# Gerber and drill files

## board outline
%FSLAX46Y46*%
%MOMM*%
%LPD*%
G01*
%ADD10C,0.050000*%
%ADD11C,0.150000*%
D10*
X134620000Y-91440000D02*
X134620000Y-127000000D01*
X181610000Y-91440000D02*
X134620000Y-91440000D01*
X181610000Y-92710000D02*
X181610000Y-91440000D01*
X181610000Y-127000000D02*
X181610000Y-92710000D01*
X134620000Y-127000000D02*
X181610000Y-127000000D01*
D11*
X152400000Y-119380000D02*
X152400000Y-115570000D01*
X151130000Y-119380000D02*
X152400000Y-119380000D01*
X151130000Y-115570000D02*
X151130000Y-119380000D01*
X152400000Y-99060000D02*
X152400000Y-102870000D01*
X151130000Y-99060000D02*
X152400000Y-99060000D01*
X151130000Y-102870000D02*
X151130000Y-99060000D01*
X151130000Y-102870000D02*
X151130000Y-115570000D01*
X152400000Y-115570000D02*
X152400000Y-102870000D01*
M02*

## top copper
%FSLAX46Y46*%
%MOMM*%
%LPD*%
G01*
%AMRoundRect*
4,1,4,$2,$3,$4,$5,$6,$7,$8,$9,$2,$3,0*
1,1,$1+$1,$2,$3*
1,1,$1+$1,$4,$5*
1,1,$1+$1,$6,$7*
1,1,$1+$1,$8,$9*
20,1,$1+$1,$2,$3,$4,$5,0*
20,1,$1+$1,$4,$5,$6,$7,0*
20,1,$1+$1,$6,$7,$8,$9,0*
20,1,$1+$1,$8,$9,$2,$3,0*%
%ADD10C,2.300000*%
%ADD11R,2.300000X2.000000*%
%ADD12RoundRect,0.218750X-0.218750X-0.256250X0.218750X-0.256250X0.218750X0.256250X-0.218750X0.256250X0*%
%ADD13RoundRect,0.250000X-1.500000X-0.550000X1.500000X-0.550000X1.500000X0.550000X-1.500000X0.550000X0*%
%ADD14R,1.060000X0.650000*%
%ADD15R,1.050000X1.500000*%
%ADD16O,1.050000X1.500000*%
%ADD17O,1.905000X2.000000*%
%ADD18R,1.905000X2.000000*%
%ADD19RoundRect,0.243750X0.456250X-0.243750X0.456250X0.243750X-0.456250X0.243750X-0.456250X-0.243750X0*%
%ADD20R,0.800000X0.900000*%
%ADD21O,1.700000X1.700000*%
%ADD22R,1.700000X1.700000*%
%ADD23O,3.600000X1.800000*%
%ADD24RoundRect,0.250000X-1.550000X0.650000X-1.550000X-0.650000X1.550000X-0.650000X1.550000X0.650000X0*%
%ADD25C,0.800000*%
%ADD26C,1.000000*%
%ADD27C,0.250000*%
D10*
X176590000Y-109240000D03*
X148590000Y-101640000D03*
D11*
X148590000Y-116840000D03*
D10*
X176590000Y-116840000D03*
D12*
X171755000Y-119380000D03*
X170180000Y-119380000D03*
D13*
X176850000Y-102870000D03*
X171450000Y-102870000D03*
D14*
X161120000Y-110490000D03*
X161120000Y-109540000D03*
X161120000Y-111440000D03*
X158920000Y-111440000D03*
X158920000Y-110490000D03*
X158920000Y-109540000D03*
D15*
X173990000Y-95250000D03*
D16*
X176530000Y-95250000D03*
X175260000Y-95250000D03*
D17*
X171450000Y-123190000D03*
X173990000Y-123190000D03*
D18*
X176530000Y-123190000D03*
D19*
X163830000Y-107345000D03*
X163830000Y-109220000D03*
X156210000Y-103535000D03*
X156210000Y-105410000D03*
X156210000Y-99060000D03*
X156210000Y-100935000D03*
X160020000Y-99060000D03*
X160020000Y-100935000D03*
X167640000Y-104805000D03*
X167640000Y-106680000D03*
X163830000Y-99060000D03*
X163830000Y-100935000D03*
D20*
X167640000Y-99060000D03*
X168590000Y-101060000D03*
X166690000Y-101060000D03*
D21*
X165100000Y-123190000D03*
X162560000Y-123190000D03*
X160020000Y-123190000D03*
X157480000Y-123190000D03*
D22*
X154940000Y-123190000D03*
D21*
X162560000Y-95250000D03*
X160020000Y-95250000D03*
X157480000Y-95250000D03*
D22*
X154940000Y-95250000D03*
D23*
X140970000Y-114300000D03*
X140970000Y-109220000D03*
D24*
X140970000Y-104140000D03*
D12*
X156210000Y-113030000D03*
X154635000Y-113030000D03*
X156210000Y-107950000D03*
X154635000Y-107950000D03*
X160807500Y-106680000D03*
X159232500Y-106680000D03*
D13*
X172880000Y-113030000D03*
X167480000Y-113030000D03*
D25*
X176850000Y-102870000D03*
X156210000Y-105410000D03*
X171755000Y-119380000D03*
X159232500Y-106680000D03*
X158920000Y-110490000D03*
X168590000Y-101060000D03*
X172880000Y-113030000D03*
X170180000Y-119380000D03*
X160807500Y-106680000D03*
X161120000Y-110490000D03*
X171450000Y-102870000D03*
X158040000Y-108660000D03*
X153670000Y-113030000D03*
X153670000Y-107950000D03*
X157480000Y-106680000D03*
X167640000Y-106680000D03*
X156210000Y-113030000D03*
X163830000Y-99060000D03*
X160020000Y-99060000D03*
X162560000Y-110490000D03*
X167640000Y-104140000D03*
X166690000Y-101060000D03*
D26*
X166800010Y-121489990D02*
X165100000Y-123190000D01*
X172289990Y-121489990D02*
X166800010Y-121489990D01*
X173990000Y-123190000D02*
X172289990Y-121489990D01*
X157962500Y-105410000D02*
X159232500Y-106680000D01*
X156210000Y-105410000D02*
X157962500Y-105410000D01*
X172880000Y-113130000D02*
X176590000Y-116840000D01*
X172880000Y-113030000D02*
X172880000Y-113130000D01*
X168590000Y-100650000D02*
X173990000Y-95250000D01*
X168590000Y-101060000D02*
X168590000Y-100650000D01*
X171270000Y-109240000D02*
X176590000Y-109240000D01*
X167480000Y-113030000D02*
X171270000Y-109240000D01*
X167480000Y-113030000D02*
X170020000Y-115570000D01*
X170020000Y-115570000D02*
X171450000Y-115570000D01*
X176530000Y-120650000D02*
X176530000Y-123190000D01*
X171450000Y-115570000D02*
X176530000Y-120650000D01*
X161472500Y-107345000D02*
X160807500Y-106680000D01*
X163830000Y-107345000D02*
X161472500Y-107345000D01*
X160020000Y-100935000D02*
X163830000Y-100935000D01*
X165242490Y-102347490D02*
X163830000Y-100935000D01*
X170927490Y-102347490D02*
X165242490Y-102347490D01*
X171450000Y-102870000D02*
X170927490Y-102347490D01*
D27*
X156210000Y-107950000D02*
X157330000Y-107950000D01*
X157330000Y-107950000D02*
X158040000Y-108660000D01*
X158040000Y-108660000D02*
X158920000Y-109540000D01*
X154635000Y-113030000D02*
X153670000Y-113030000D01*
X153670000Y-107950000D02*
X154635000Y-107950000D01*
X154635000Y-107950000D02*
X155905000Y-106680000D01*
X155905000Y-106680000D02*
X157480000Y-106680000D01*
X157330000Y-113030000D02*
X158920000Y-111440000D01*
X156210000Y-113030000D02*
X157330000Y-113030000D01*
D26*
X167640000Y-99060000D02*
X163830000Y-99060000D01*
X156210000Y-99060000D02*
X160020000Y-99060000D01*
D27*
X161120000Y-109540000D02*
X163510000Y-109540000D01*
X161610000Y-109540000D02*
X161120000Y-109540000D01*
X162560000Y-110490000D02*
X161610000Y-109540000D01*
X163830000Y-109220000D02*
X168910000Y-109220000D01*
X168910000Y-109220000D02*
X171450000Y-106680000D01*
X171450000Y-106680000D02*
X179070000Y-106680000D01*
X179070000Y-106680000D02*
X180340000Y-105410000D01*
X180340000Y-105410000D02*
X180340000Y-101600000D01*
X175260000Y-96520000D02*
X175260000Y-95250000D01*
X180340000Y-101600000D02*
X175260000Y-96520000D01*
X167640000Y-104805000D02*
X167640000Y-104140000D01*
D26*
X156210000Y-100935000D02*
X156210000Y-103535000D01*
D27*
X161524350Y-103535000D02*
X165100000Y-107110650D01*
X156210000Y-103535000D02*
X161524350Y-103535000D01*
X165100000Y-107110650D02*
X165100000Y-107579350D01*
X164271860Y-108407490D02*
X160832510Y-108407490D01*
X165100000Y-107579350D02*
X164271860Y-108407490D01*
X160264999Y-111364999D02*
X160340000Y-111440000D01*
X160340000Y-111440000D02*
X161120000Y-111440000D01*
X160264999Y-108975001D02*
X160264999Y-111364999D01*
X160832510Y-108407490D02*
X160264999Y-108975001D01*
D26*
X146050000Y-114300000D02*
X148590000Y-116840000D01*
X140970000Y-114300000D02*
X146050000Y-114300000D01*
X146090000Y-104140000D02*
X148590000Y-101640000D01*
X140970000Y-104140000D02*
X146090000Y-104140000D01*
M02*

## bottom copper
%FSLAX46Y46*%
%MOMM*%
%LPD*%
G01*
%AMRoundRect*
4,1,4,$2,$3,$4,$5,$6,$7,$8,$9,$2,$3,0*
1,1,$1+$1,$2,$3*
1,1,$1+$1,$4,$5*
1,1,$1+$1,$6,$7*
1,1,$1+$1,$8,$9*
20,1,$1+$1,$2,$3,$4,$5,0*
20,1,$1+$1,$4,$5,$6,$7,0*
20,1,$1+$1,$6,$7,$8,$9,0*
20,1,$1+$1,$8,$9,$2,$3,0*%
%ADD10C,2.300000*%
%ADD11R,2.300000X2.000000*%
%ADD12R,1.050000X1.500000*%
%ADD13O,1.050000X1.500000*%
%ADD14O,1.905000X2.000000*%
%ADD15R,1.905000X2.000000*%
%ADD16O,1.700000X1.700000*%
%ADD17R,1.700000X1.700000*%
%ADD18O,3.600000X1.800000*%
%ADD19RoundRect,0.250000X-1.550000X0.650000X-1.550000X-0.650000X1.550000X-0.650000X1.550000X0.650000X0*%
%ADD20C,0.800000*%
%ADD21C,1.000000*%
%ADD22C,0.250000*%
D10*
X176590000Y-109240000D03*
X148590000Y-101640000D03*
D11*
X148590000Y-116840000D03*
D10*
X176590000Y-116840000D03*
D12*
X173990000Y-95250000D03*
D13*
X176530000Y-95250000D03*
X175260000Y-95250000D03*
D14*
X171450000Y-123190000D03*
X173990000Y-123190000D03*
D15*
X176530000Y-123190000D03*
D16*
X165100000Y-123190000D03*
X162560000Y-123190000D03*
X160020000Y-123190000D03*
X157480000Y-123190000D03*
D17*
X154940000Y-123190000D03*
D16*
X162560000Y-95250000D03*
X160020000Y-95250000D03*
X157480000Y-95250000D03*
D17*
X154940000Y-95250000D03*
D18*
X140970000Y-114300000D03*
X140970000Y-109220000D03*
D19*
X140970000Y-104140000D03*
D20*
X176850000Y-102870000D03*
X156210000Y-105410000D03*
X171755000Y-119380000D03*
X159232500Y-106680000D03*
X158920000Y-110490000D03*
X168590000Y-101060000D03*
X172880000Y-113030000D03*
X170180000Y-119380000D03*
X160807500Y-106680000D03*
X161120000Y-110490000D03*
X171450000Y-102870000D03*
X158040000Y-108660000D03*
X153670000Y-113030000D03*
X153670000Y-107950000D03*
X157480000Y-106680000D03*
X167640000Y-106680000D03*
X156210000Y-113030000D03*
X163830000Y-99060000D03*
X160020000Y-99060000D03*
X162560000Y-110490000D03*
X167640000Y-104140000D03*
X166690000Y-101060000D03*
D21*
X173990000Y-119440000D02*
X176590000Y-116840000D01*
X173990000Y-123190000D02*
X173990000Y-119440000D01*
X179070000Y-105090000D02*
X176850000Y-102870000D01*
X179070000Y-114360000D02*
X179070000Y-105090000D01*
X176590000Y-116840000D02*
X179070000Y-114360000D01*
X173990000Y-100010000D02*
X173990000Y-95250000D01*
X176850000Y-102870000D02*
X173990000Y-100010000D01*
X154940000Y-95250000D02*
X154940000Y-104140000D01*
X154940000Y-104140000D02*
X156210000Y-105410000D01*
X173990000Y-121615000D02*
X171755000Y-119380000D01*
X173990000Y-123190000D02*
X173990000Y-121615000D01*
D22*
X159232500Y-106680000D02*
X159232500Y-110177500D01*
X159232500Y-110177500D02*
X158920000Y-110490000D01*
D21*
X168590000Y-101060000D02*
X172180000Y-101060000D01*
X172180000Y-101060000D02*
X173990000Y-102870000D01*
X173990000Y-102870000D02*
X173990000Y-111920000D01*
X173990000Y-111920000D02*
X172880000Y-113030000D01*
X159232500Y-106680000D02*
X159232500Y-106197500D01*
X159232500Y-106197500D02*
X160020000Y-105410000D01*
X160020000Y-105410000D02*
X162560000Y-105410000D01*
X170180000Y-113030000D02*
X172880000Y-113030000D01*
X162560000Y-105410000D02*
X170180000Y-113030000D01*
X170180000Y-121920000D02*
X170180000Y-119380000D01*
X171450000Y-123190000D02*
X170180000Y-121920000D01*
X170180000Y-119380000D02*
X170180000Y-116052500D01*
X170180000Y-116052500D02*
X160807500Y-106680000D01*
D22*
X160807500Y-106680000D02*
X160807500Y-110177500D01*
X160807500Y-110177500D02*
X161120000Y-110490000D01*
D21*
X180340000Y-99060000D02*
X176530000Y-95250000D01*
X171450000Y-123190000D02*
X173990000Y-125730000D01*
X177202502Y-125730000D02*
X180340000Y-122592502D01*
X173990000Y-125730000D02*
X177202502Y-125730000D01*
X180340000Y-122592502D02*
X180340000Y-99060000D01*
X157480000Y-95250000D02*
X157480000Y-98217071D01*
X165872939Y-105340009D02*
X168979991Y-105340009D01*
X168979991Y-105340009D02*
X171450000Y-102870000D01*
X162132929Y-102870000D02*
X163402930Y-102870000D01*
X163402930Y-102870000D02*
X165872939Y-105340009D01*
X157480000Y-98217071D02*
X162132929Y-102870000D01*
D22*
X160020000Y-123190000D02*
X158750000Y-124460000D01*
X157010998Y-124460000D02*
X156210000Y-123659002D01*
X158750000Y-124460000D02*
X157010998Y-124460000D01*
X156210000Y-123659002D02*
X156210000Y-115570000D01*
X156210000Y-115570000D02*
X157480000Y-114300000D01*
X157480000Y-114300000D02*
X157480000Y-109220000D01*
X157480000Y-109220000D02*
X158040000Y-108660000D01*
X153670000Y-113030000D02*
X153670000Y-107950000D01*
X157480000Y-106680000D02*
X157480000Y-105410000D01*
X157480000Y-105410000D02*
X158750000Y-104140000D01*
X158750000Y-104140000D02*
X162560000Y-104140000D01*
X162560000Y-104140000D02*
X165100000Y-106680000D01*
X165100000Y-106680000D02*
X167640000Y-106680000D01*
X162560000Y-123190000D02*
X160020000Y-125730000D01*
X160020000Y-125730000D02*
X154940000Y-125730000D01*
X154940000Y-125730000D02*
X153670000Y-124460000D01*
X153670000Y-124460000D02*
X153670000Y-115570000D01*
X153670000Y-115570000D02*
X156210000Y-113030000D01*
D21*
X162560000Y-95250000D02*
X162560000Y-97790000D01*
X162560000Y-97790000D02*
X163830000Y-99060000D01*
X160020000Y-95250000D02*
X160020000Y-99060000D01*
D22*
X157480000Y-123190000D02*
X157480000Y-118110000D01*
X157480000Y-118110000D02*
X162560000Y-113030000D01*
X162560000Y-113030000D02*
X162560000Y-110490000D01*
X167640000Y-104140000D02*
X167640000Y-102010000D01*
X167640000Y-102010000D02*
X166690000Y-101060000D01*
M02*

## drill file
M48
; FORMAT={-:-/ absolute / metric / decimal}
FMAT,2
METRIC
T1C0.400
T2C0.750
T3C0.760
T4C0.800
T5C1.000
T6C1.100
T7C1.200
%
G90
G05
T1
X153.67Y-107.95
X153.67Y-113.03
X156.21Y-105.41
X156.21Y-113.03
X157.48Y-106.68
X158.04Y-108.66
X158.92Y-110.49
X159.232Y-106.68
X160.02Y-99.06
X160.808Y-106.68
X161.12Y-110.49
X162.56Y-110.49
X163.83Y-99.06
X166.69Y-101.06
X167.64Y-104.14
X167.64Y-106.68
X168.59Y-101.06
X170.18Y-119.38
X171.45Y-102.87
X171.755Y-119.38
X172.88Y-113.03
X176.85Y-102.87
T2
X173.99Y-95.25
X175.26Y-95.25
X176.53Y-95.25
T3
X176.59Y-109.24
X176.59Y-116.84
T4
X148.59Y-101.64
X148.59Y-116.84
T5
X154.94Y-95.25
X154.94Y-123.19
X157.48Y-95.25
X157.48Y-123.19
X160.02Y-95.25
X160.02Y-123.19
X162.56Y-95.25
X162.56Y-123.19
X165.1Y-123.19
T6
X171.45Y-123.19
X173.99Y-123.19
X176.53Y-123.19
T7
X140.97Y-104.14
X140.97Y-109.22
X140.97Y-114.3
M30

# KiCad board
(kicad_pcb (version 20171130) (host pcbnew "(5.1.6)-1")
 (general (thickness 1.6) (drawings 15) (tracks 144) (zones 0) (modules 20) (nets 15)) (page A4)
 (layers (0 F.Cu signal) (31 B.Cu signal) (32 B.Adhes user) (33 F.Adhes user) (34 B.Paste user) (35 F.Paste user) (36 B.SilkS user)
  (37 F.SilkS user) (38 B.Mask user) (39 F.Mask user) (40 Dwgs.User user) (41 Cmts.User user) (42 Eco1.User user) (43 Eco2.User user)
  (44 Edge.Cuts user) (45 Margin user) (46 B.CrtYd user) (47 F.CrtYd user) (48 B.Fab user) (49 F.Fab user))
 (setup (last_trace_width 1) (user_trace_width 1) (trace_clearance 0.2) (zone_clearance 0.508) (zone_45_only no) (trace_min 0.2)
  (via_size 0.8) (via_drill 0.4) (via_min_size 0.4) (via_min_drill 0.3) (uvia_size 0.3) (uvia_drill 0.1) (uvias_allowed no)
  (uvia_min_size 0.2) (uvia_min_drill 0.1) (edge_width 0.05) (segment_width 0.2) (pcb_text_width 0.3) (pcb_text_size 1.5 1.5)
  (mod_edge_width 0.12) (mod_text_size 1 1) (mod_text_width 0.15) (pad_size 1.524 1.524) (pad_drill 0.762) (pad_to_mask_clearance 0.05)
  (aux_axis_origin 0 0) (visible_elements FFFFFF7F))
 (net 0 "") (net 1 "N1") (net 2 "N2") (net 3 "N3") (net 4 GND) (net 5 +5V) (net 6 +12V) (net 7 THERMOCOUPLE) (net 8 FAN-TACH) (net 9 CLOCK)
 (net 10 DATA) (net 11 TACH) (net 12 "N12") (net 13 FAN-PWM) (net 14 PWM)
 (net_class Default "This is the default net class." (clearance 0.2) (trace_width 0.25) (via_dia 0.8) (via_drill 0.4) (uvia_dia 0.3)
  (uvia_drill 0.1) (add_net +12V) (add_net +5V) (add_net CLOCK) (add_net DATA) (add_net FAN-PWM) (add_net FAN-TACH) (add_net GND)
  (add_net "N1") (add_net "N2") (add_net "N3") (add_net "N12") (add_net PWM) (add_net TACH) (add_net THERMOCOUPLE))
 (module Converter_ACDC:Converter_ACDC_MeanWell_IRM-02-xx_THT (layer B.Cu) (at 148.59 116.84)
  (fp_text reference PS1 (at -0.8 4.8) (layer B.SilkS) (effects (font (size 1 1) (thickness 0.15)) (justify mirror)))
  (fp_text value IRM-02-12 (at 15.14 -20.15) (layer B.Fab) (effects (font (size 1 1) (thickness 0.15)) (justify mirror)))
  (pad 4 thru_hole circle (at 28 -7.6) (size 2.3 2.3) (drill 0.76) (layers *.Cu *.Mask) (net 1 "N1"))
  (pad 2 thru_hole circle (at 0 -15.2) (size 2.3 2.3) (drill 0.8) (layers *.Cu *.Mask) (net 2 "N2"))
  (pad 1 thru_hole rect (at 0 0) (size 2.3 2) (drill 0.8) (layers *.Cu *.Mask) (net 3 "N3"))
  (pad 3 thru_hole circle (at 28 0) (size 2.3 2.3) (drill 0.76) (layers *.Cu *.Mask) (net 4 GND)))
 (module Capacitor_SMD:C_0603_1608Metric (layer F.Cu) (at 170.9675 119.38)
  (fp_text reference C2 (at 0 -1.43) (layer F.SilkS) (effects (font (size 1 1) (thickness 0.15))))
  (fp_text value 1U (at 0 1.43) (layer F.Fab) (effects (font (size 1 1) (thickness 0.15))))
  (pad 2 smd roundrect (at 0.7875 0) (size 0.875 0.95) (layers F.Cu F.Paste F.Mask) (roundrect_rratio 0.25) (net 4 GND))
  (pad 1 smd roundrect (at -0.7875 0) (size 0.875 0.95) (layers F.Cu F.Paste F.Mask) (roundrect_rratio 0.25) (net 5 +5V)))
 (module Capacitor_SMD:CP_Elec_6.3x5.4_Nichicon (layer F.Cu) (at 174.15 102.87)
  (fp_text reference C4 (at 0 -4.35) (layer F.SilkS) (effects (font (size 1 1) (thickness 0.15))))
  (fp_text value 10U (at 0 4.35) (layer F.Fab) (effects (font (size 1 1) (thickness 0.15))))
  (pad 2 smd roundrect (at 2.7 0) (size 3.5 1.6) (layers F.Cu F.Paste F.Mask) (roundrect_rratio 0.15625) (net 4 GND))
  (pad 1 smd roundrect (at -2.7 0) (size 3.5 1.6) (layers F.Cu F.Paste F.Mask) (roundrect_rratio 0.15625) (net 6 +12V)))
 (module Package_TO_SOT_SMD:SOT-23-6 (layer F.Cu) (at 160.02 110.49)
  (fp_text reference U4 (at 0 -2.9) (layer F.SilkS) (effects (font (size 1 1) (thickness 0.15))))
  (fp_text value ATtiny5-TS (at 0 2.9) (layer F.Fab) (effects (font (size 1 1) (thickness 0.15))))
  (pad 5 smd rect (at 1.1 0) (size 1.06 0.65) (layers F.Cu F.Paste F.Mask) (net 5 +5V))
  (pad 6 smd rect (at 1.1 -0.95) (size 1.06 0.65) (layers F.Cu F.Paste F.Mask) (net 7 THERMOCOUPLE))
  (pad 4 smd rect (at 1.1 0.95) (size 1.06 0.65) (layers F.Cu F.Paste F.Mask) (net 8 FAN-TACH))
  (pad 3 smd rect (at -1.1 0.95) (size 1.06 0.65) (layers F.Cu F.Paste F.Mask) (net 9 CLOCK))
  (pad 2 smd rect (at -1.1 0) (size 1.06 0.65) (layers F.Cu F.Paste F.Mask) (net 4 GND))
  (pad 1 smd rect (at -1.1 -0.95) (size 1.06 0.65) (layers F.Cu F.Paste F.Mask) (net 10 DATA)))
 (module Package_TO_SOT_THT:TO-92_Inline (layer F.Cu) (at 173.99 95.25)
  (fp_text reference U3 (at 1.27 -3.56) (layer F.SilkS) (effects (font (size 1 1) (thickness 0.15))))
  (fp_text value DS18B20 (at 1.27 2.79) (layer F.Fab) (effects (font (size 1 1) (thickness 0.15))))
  (pad 1 thru_hole rect (at 0 0) (size 1.05 1.5) (drill 0.75) (layers *.Cu *.Mask) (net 4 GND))
  (pad 3 thru_hole oval (at 2.54 0) (size 1.05 1.5) (drill 0.75) (layers *.Cu *.Mask) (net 5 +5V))
  (pad 2 thru_hole oval (at 1.27 0) (size 1.05 1.5) (drill 0.75) (layers *.Cu *.Mask) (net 7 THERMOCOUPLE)))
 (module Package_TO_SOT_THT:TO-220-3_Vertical (layer F.Cu) (at 176.53 123.19 180)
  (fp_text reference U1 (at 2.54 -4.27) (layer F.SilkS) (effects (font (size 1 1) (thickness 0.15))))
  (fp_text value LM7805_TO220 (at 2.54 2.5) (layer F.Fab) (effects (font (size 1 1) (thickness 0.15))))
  (pad 3 thru_hole oval (at 5.08 0 180) (size 1.905 2) (drill 1.1) (layers *.Cu *.Mask) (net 5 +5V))
  (pad 2 thru_hole oval (at 2.54 0 180) (size 1.905 2) (drill 1.1) (layers *.Cu *.Mask) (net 4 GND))
  (pad 1 thru_hole rect (at 0 0 180) (size 1.905 2) (drill 1.1) (layers *.Cu *.Mask) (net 1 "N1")))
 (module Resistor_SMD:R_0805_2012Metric (layer F.Cu) (at 163.83 108.2825 90)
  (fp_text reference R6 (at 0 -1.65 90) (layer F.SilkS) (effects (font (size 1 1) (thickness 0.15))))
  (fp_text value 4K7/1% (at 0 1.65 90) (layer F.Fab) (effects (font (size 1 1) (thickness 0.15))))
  (pad 2 smd roundrect (at 0.9375 0 90) (size 0.975 1.4) (layers F.Cu F.Paste F.Mask) (roundrect_rratio 0.25) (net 5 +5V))
  (pad 1 smd roundrect (at -0.9375 0 90) (size 0.975 1.4) (layers F.Cu F.Paste F.Mask) (roundrect_rratio 0.25) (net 7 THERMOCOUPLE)))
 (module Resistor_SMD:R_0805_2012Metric (layer F.Cu) (at 156.21 104.4725 90)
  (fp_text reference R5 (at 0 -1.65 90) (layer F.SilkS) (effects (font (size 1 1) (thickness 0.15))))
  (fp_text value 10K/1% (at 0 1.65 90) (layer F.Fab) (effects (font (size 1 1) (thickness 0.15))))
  (pad 2 smd roundrect (at 0.9375 0 90) (size 0.975 1.4) (layers F.Cu F.Paste F.Mask) (roundrect_rratio 0.25) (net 8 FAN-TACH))
  (pad 1 smd roundrect (at -0.9375 0 90) (size 0.975 1.4) (layers F.Cu F.Paste F.Mask) (roundrect_rratio 0.25) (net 4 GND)))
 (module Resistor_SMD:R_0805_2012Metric (layer F.Cu) (at 156.21 99.9975 90)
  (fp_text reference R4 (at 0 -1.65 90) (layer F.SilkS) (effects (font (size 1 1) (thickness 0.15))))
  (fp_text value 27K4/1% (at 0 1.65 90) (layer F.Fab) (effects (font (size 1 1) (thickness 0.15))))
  (pad 2 smd roundrect (at 0.9375 0 90) (size 0.975 1.4) (layers F.Cu F.Paste F.Mask) (roundrect_rratio 0.25) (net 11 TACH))
  (pad 1 smd roundrect (at -0.9375 0 90) (size 0.975 1.4) (layers F.Cu F.Paste F.Mask) (roundrect_rratio 0.25) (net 8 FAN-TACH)))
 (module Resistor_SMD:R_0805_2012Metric (layer F.Cu) (at 160.02 99.9975 90)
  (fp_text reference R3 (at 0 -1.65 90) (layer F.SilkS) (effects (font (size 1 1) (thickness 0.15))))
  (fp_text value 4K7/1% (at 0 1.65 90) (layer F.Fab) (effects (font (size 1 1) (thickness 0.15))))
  (pad 2 smd roundrect (at 0.9375 0 90) (size 0.975 1.4) (layers F.Cu F.Paste F.Mask) (roundrect_rratio 0.25) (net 11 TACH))
  (pad 1 smd roundrect (at -0.9375 0 90) (size 0.975 1.4) (layers F.Cu F.Paste F.Mask) (roundrect_rratio 0.25) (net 6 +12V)))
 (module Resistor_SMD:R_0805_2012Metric (layer F.Cu) (at 167.64 105.7425 90)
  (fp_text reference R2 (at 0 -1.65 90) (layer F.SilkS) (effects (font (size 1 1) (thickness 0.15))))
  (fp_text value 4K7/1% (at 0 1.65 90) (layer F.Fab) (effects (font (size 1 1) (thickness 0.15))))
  (pad 2 smd roundrect (at 0.9375 0 90) (size 0.975 1.4) (layers F.Cu F.Paste F.Mask) (roundrect_rratio 0.25) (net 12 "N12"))
  (pad 1 smd roundrect (at -0.9375 0 90) (size 0.975 1.4) (layers F.Cu F.Paste F.Mask) (roundrect_rratio 0.25) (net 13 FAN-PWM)))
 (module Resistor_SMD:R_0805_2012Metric (layer F.Cu) (at 163.83 99.9975 90)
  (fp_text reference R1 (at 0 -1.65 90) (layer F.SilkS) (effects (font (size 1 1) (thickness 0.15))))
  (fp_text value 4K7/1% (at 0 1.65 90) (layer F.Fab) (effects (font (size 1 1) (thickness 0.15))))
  (pad 2 smd roundrect (at 0.9375 0 90) (size 0.975 1.4) (layers F.Cu F.Paste F.Mask) (roundrect_rratio 0.25) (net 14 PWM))
  (pad 1 smd roundrect (at -0.9375 0 90) (size 0.975 1.4) (layers F.Cu F.Paste F.Mask) (roundrect_rratio 0.25) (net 6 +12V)))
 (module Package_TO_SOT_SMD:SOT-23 (layer F.Cu) (at 167.64 100.06 90)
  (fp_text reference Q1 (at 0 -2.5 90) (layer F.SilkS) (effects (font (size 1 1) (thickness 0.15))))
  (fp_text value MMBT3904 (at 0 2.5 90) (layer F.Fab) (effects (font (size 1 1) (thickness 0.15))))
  (pad 3 smd rect (at 1 0 90) (size 0.9 0.8) (layers F.Cu F.Paste F.Mask) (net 14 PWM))
  (pad 2 smd rect (at -1 0.95 90) (size 0.9 0.8) (layers F.Cu F.Paste F.Mask) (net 4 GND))
  (pad 1 smd rect (at -1 -0.95 90) (size 0.9 0.8) (layers F.Cu F.Paste F.Mask) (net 12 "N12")))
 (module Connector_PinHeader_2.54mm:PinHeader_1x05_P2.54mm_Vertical (layer F.Cu) (at 154.94 123.19 90)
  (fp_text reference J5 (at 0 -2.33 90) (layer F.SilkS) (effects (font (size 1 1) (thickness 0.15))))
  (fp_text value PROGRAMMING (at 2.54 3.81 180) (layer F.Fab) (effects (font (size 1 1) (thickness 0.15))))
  (pad 5 thru_hole oval (at 0 10.16 90) (size 1.7 1.7) (drill 1) (layers *.Cu *.Mask) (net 4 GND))
  (pad 4 thru_hole oval (at 0 7.62 90) (size 1.7 1.7) (drill 1) (layers *.Cu *.Mask) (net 9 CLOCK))
  (pad 3 thru_hole oval (at 0 5.08 90) (size 1.7 1.7) (drill 1) (layers *.Cu *.Mask) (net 10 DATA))
  (pad 2 thru_hole oval (at 0 2.54 90) (size 1.7 1.7) (drill 1) (layers *.Cu *.Mask) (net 7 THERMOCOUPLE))
  (pad 1 thru_hole rect (at 0 0 90) (size 1.7 1.7) (drill 1) (layers *.Cu *.Mask)))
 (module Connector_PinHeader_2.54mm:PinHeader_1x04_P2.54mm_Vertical (layer F.Cu) (at 154.94 95.25 90)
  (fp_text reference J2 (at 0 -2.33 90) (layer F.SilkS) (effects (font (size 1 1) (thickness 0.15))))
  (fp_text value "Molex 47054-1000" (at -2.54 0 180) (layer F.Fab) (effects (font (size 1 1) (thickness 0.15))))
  (pad 4 thru_hole oval (at 0 7.62 90) (size 1.7 1.7) (drill 1) (layers *.Cu *.Mask) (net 14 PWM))
  (pad 3 thru_hole oval (at 0 5.08 90) (size 1.7 1.7) (drill 1) (layers *.Cu *.Mask) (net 11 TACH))
  (pad 2 thru_hole oval (at 0 2.54 90) (size 1.7 1.7) (drill 1) (layers *.Cu *.Mask) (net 6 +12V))
  (pad 1 thru_hole rect (at 0 0 90) (size 1.7 1.7) (drill 1) (layers *.Cu *.Mask) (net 4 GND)))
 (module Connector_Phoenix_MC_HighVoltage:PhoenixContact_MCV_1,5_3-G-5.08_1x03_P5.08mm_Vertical (layer B.Cu) (at 140.97 104.14 270)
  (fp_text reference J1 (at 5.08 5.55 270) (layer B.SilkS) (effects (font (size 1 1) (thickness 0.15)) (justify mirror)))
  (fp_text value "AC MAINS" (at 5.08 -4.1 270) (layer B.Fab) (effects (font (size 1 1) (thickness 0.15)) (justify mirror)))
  (pad 3 thru_hole oval (at 10.16 0 270) (size 1.8 3.6) (drill 1.2) (layers *.Cu *.Mask) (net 3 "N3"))
  (pad 2 thru_hole oval (at 5.08 0 270) (size 1.8 3.6) (drill 1.2) (layers *.Cu *.Mask))
  (pad 1 thru_hole roundrect (at 0 0 270) (size 1.8 3.6) (drill 1.2) (layers *.Cu *.Mask) (roundrect_rratio 0.138889) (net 2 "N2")))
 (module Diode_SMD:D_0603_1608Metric (layer F.Cu) (at 155.4225 113.03)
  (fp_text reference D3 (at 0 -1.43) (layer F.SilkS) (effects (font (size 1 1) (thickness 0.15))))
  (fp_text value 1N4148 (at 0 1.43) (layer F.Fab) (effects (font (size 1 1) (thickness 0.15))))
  (pad 2 smd roundrect (at 0.7875 0) (size 0.875 0.95) (layers F.Cu F.Paste F.Mask) (roundrect_rratio 0.25) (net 9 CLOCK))
  (pad 1 smd roundrect (at -0.7875 0) (size 0.875 0.95) (layers F.Cu F.Paste F.Mask) (roundrect_rratio 0.25) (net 13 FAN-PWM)))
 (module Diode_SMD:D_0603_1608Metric (layer F.Cu) (at 155.4225 107.95)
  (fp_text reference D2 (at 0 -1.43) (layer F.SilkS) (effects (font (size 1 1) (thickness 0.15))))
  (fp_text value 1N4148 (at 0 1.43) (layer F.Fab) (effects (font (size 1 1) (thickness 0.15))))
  (pad 2 smd roundrect (at 0.7875 0) (size 0.875 0.95) (layers F.Cu F.Paste F.Mask) (roundrect_rratio 0.25) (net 10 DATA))
  (pad 1 smd roundrect (at -0.7875 0) (size 0.875 0.95) (layers F.Cu F.Paste F.Mask) (roundrect_rratio 0.25) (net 13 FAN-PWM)))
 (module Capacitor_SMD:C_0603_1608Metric (layer F.Cu) (at 160.02 106.68)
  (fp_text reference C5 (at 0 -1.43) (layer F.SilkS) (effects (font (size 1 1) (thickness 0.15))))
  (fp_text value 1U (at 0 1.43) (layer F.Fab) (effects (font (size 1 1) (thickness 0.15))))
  (pad 2 smd roundrect (at 0.7875 0) (size 0.875 0.95) (layers F.Cu F.Paste F.Mask) (roundrect_rratio 0.25) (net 5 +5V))
  (pad 1 smd roundrect (at -0.7875 0) (size 0.875 0.95) (layers F.Cu F.Paste F.Mask) (roundrect_rratio 0.25) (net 4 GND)))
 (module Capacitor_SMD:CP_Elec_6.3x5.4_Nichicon (layer F.Cu) (at 170.18 113.03)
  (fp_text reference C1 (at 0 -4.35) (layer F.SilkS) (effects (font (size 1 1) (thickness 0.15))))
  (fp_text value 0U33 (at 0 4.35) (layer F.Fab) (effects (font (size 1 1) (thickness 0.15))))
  (pad 2 smd roundrect (at 2.7 0) (size 3.5 1.6) (layers F.Cu F.Paste F.Mask) (roundrect_rratio 0.15625) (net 4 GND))
  (pad 1 smd roundrect (at -2.7 0) (size 3.5 1.6) (layers F.Cu F.Paste F.Mask) (roundrect_rratio 0.15625) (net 1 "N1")))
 (gr_line (start 134.62 91.44) (end 134.62 127) (layer Edge.Cuts) (width 0.05))
 (gr_line (start 181.61 91.44) (end 134.62 91.44) (layer Edge.Cuts) (width 0.05))
 (gr_line (start 181.61 92.71) (end 181.61 91.44) (layer Edge.Cuts) (width 0.05))
 (gr_line (start 181.61 127) (end 181.61 92.71) (layer Edge.Cuts) (width 0.05))
 (gr_line (start 134.62 127) (end 181.61 127) (layer Edge.Cuts) (width 0.05))
 (gr_line (start 152.4 119.38) (end 152.4 115.57) (layer Edge.Cuts) (width 0.15))
 (gr_line (start 151.13 119.38) (end 152.4 119.38) (layer Edge.Cuts) (width 0.15))
 (gr_line (start 151.13 115.57) (end 151.13 119.38) (layer Edge.Cuts) (width 0.15))
 (gr_line (start 152.4 99.06) (end 152.4 102.87) (layer Edge.Cuts) (width 0.15))
 (gr_line (start 151.13 99.06) (end 152.4 99.06) (layer Edge.Cuts) (width 0.15))
 (gr_line (start 151.13 102.87) (end 151.13 99.06) (layer Edge.Cuts) (width 0.15))
 (gr_line (start 151.13 102.87) (end 151.13 115.57) (layer Edge.Cuts) (width 0.15))
 (gr_line (start 152.4 115.57) (end 152.4 102.87) (layer Edge.Cuts) (width 0.15))
 (segment (start 173.99 119.44) (end 176.59 116.84) (width 1) (layer B.Cu) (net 4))
 (segment (start 173.99 123.19) (end 173.99 119.44) (width 1) (layer B.Cu) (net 4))
 (segment (start 166.80001 121.48999) (end 165.1 123.19) (width 1) (layer F.Cu) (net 4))
 (segment (start 172.28999 121.48999) (end 166.80001 121.48999) (width 1) (layer F.Cu) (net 4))
 (segment (start 173.99 123.19) (end 172.28999 121.48999) (width 1) (layer F.Cu) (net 4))
 (segment (start 179.07 105.09) (end 176.85 102.87) (width 1) (layer B.Cu) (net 4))
 (segment (start 179.07 114.36) (end 179.07 105.09) (width 1) (layer B.Cu) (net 4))
 (segment (start 176.59 116.84) (end 179.07 114.36) (width 1) (layer B.Cu) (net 4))
 (via (at 176.85 102.87) (size 0.8) (drill 0.4) (layers F.Cu B.Cu) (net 4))
 (segment (start 173.99 100.01) (end 173.99 95.25) (width 1) (layer B.Cu) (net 4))
 (segment (start 176.85 102.87) (end 173.99 100.01) (width 1) (layer B.Cu) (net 4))
 (via (at 156.21 105.41) (size 0.8) (drill 0.4) (layers F.Cu B.Cu) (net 4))
 (segment (start 154.94 95.25) (end 154.94 104.14) (width 1) (layer B.Cu) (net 4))
 (segment (start 154.94 104.14) (end 156.21 105.41) (width 1) (layer B.Cu) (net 4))
 (segment (start 157.9625 105.41) (end 159.2325 106.68) (width 1) (layer F.Cu) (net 4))
 (segment (start 156.21 105.41) (end 157.9625 105.41) (width 1) (layer F.Cu) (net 4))
 (segment (start 173.99 121.615) (end 171.755 119.38) (width 1) (layer B.Cu) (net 4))
 (via (at 171.755 119.38) (size 0.8) (drill 0.4) (layers F.Cu B.Cu) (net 4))
 (segment (start 173.99 123.19) (end 173.99 121.615) (width 1) (layer B.Cu) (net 4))
 (segment (start 172.88 113.13) (end 176.59 116.84) (width 1) (layer F.Cu) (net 4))
 (segment (start 172.88 113.03) (end 172.88 113.13) (width 1) (layer F.Cu) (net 4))
 (segment (start 168.59 100.65) (end 173.99 95.25) (width 1) (layer F.Cu) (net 4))
 (segment (start 168.59 101.06) (end 168.59 100.65) (width 1) (layer F.Cu) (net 4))
 (via (at 159.2325 106.68) (size 0.8) (drill 0.4) (layers F.Cu B.Cu) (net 4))
 (segment (start 159.2325 106.68) (end 159.2325 110.1775) (width 0.25) (layer B.Cu) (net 4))
 (via (at 158.92 110.49) (size 0.8) (drill 0.4) (layers F.Cu B.Cu) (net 4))
 (segment (start 159.2325 110.1775) (end 158.92 110.49) (width 0.25) (layer B.Cu) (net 4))
 (via (at 168.59 101.06) (size 0.8) (drill 0.4) (layers F.Cu B.Cu) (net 4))
 (segment (start 168.59 101.06) (end 172.18 101.06) (width 1) (layer B.Cu) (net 4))
 (segment (start 172.18 101.06) (end 173.99 102.87) (width 1) (layer B.Cu) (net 4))
 (via (at 172.88 113.03) (size 0.8) (drill 0.4) (layers F.Cu B.Cu) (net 4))
 (segment (start 173.99 102.87) (end 173.99 111.92) (width 1) (layer B.Cu) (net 4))
 (segment (start 173.99 111.92) (end 172.88 113.03) (width 1) (layer B.Cu) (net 4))
 (segment (start 159.2325 106.68) (end 159.2325 106.1975) (width 1) (layer B.Cu) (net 4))
 (segment (start 159.2325 106.1975) (end 160.02 105.41) (width 1) (layer B.Cu) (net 4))
 (segment (start 160.02 105.41) (end 162.56 105.41) (width 1) (layer B.Cu) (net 4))
 (segment (start 170.18 113.03) (end 172.88 113.03) (width 1) (layer B.Cu) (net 4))
 (segment (start 162.56 105.41) (end 170.18 113.03) (width 1) (layer B.Cu) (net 4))
 (segment (start 171.27 109.24) (end 176.59 109.24) (width 1) (layer F.Cu) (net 1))
 (segment (start 167.48 113.03) (end 171.27 109.24) (width 1) (layer F.Cu) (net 1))
 (segment (start 167.48 113.03) (end 170.02 115.57) (width 1) (layer F.Cu) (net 1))
 (segment (start 170.02 115.57) (end 171.45 115.57) (width 1) (layer F.Cu) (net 1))
 (segment (start 176.53 120.65) (end 176.53 123.19) (width 1) (layer F.Cu) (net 1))
 (segment (start 171.45 115.57) (end 176.53 120.65) (width 1) (layer F.Cu) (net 1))
 (segment (start 161.4725 107.345) (end 160.8075 106.68) (width 1) (layer F.Cu) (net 5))
 (segment (start 163.83 107.345) (end 161.4725 107.345) (width 1) (layer F.Cu) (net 5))
 (via (at 170.18 119.38) (size 0.8) (drill 0.4) (layers F.Cu B.Cu) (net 5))
 (segment (start 170.18 121.92) (end 170.18 119.38) (width 1) (layer B.Cu) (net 5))
 (segment (start 171.45 123.19) (end 170.18 121.92) (width 1) (layer B.Cu) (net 5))
 (via (at 160.8075 106.68) (size 0.8) (drill 0.4) (layers F.Cu B.Cu) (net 5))
 (segment (start 170.18 119.38) (end 170.18 116.0525) (width 1) (layer B.Cu) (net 5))
 (segment (start 170.18 116.0525) (end 160.8075 106.68) (width 1) (layer B.Cu) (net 5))
 (via (at 161.12 110.49) (size 0.8) (drill 0.4) (layers F.Cu B.Cu) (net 5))
 (segment (start 160.8075 106.68) (end 160.8075 110.1775) (width 0.25) (layer B.Cu) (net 5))
 (segment (start 160.8075 110.1775) (end 161.12 110.49) (width 0.25) (layer B.Cu) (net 5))
 (segment (start 180.34 99.06) (end 176.53 95.25) (width 1) (layer B.Cu) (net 5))
 (segment (start 171.45 123.19) (end 173.99 125.73) (width 1) (layer B.Cu) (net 5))
 (segment (start 177.202502 125.73) (end 180.34 122.592502) (width 1) (layer B.Cu) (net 5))
 (segment (start 173.99 125.73) (end 177.202502 125.73) (width 1) (layer B.Cu) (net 5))
 (segment (start 180.34 122.592502) (end 180.34 99.06) (width 1) (layer B.Cu) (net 5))
 (segment (start 160.02 100.935) (end 163.83 100.935) (width 1) (layer F.Cu) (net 6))
 (segment (start 165.24249 102.34749) (end 163.83 100.935) (width 1) (layer F.Cu) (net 6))
 (segment (start 170.92749 102.34749) (end 165.24249 102.34749) (width 1) (layer F.Cu) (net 6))
 (segment (start 171.45 102.87) (end 170.92749 102.34749) (width 1) (layer F.Cu) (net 6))
 (via (at 171.45 102.87) (size 0.8) (drill 0.4) (layers F.Cu B.Cu) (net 6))
 (segment (start 157.48 95.25) (end 157.48 98.217071) (width 1) (layer B.Cu) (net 6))
 (segment (start 165.872939 105.340009) (end 168.979991 105.340009) (width 1) (layer B.Cu) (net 6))
 (segment (start 168.979991 105.340009) (end 171.45 102.87) (width 1) (layer B.Cu) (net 6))
 (segment (start 162.132929 102.87) (end 163.40293 102.87) (width 1) (layer B.Cu) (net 6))
 (segment (start 163.40293 102.87) (end 165.872939 105.340009) (width 1) (layer B.Cu) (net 6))
 (segment (start 157.48 98.217071) (end 162.132929 102.87) (width 1) (layer B.Cu) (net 6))
 (segment (start 156.21 107.95) (end 157.33 107.95) (width 0.25) (layer F.Cu) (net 10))
 (segment (start 160.02 123.19) (end 158.75 124.46) (width 0.25) (layer B.Cu) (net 10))
 (segment (start 157.010998 124.46) (end 156.21 123.659002) (width 0.25) (layer B.Cu) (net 10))
 (segment (start 158.75 124.46) (end 157.010998 124.46) (width 0.25) (layer B.Cu) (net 10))
 (segment (start 156.21 123.659002) (end 156.21 115.57) (width 0.25) (layer B.Cu) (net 10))
 (segment (start 156.21 115.57) (end 157.48 114.3) (width 0.25) (layer B.Cu) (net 10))
 (segment (start 157.48 114.3) (end 157.48 109.22) (width 0.25) (layer B.Cu) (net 10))
 (via (at 158.04 108.66) (size 0.8) (drill 0.4) (layers F.Cu B.Cu) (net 10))
 (segment (start 157.48 109.22) (end 158.04 108.66) (width 0.25) (layer B.Cu) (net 10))
 (segment (start 157.33 107.95) (end 158.04 108.66) (width 0.25) (layer F.Cu) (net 10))
 (segment (start 158.04 108.66) (end 158.92 109.54) (width 0.25) (layer F.Cu) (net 10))
 (via (at 153.67 113.03) (size 0.8) (drill 0.4) (layers F.Cu B.Cu) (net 13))
 (segment (start 154.635 113.03) (end 153.67 113.03) (width 0.25) (layer F.Cu) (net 13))
 (via (at 153.67 107.95) (size 0.8) (drill 0.4) (layers F.Cu B.Cu) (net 13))
 (segment (start 153.67 113.03) (end 153.67 107.95) (width 0.25) (layer B.Cu) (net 13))
 (segment (start 153.67 107.95) (end 154.635 107.95) (width 0.25) (layer F.Cu) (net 13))
 (segment (start 154.635 107.95) (end 155.905 106.68) (width 0.25) (layer F.Cu) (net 13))
 (via (at 157.48 106.68) (size 0.8) (drill 0.4) (layers F.Cu B.Cu) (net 13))
 (segment (start 155.905 106.68) (end 157.48 106.68) (width 0.25) (layer F.Cu) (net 13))
 (segment (start 157.48 106.68) (end 157.48 105.41) (width 0.25) (layer B.Cu) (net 13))
 (segment (start 157.48 105.41) (end 158.75 104.14) (width 0.25) (layer B.Cu) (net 13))
 (segment (start 158.75 104.14) (end 162.56 104.14) (width 0.25) (layer B.Cu) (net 13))
 (segment (start 162.56 104.14) (end 165.1 106.68) (width 0.25) (layer B.Cu) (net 13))
 (segment (start 165.1 106.68) (end 167.64 106.68) (width 0.25) (layer B.Cu) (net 13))
 (via (at 167.64 106.68) (size 0.8) (drill 0.4) (layers F.Cu B.Cu) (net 13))
 (segment (start 157.33 113.03) (end 158.92 111.44) (width 0.25) (layer F.Cu) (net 9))
 (segment (start 156.21 113.03) (end 157.33 113.03) (width 0.25) (layer F.Cu) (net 9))
 (segment (start 162.56 123.19) (end 160.02 125.73) (width 0.25) (layer B.Cu) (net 9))
 (segment (start 160.02 125.73) (end 154.94 125.73) (width 0.25) (layer B.Cu) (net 9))
 (segment (start 154.94 125.73) (end 153.67 124.46) (width 0.25) (layer B.Cu) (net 9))
 (segment (start 153.67 124.46) (end 153.67 115.57) (width 0.25) (layer B.Cu) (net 9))
 (via (at 156.21 113.03) (size 0.8) (drill 0.4) (layers F.Cu B.Cu) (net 9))
 (segment (start 153.67 115.57) (end 156.21 113.03) (width 0.25) (layer B.Cu) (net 9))
 (via (at 163.83 99.06) (size 0.8) (drill 0.4) (layers F.Cu B.Cu) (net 14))
 (segment (start 162.56 95.25) (end 162.56 97.79) (width 1) (layer B.Cu) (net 14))
 (segment (start 162.56 97.79) (end 163.83 99.06) (width 1) (layer B.Cu) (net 14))
 (segment (start 167.64 99.06) (end 163.83 99.06) (width 1) (layer F.Cu) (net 14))
 (segment (start 156.21 99.06) (end 160.02 99.06) (width 1) (layer F.Cu) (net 11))
 (via (at 160.02 99.06) (size 0.8) (drill 0.4) (layers F.Cu B.Cu) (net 11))
 (segment (start 160.02 95.25) (end 160.02 99.06) (width 1) (layer B.Cu) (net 11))
 (segment (start 161.12 109.54) (end 163.51 109.54) (width 0.25) (layer F.Cu) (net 7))
 (segment (start 157.48 123.19) (end 157.48 118.11) (width 0.25) (layer B.Cu) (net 7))
 (segment (start 157.48 118.11) (end 162.56 113.03) (width 0.25) (layer B.Cu) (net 7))
 (via (at 162.56 110.49) (size 0.8) (drill 0.4) (layers F.Cu B.Cu) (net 7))
 (segment (start 162.56 113.03) (end 162.56 110.49) (width 0.25) (layer B.Cu) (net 7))
 (segment (start 161.61 109.54) (end 161.12 109.54) (width 0.25) (layer F.Cu) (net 7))
 (segment (start 162.56 110.49) (end 161.61 109.54) (width 0.25) (layer F.Cu) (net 7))
 (segment (start 163.83 109.22) (end 168.91 109.22) (width 0.25) (layer F.Cu) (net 7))
 (segment (start 168.91 109.22) (end 171.45 106.68) (width 0.25) (layer F.Cu) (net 7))
 (segment (start 171.45 106.68) (end 179.07 106.68) (width 0.25) (layer F.Cu) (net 7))
 (segment (start 179.07 106.68) (end 180.34 105.41) (width 0.25) (layer F.Cu) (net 7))
 (segment (start 180.34 105.41) (end 180.34 101.6) (width 0.25) (layer F.Cu) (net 7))
 (segment (start 175.26 96.52) (end 175.26 95.25) (width 0.25) (layer F.Cu) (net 7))
 (segment (start 180.34 101.6) (end 175.26 96.52) (width 0.25) (layer F.Cu) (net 7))
 (via (at 167.64 104.14) (size 0.8) (drill 0.4) (layers F.Cu B.Cu) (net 12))
 (segment (start 167.64 104.805) (end 167.64 104.14) (width 0.25) (layer F.Cu) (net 12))
 (via (at 166.69 101.06) (size 0.8) (drill 0.4) (layers F.Cu B.Cu) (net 12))
 (segment (start 167.64 104.14) (end 167.64 102.01) (width 0.25) (layer B.Cu) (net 12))
 (segment (start 167.64 102.01) (end 166.69 101.06) (width 0.25) (layer B.Cu) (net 12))
 (segment (start 156.21 100.935) (end 156.21 103.535) (width 1) (layer F.Cu) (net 8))
 (segment (start 161.52435 103.535) (end 165.1 107.11065) (width 0.25) (layer F.Cu) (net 8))
 (segment (start 156.21 103.535) (end 161.52435 103.535) (width 0.25) (layer F.Cu) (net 8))
 (segment (start 165.1 107.11065) (end 165.1 107.57935) (width 0.25) (layer F.Cu) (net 8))
 (segment (start 164.27186 108.40749) (end 160.83251 108.40749) (width 0.25) (layer F.Cu) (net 8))
 (segment (start 165.1 107.57935) (end 164.27186 108.40749) (width 0.25) (layer F.Cu) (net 8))
 (segment (start 160.264999 111.364999) (end 160.34 111.44) (width 0.25) (layer F.Cu) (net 8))
 (segment (start 160.34 111.44) (end 161.12 111.44) (width 0.25) (layer F.Cu) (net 8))
 (segment (start 160.264999 108.975001) (end 160.264999 111.364999) (width 0.25) (layer F.Cu) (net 8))
 (segment (start 160.83251 108.40749) (end 160.264999 108.975001) (width 0.25) (layer F.Cu) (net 8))
 (segment (start 146.05 114.3) (end 148.59 116.84) (width 1) (layer F.Cu) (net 3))
 (segment (start 140.97 114.3) (end 146.05 114.3) (width 1) (layer F.Cu) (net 3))
 (segment (start 146.09 104.14) (end 148.59 101.64) (width 1) (layer F.Cu) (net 2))
 (segment (start 140.97 104.14) (end 146.09 104.14) (width 1) (layer F.Cu) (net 2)))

